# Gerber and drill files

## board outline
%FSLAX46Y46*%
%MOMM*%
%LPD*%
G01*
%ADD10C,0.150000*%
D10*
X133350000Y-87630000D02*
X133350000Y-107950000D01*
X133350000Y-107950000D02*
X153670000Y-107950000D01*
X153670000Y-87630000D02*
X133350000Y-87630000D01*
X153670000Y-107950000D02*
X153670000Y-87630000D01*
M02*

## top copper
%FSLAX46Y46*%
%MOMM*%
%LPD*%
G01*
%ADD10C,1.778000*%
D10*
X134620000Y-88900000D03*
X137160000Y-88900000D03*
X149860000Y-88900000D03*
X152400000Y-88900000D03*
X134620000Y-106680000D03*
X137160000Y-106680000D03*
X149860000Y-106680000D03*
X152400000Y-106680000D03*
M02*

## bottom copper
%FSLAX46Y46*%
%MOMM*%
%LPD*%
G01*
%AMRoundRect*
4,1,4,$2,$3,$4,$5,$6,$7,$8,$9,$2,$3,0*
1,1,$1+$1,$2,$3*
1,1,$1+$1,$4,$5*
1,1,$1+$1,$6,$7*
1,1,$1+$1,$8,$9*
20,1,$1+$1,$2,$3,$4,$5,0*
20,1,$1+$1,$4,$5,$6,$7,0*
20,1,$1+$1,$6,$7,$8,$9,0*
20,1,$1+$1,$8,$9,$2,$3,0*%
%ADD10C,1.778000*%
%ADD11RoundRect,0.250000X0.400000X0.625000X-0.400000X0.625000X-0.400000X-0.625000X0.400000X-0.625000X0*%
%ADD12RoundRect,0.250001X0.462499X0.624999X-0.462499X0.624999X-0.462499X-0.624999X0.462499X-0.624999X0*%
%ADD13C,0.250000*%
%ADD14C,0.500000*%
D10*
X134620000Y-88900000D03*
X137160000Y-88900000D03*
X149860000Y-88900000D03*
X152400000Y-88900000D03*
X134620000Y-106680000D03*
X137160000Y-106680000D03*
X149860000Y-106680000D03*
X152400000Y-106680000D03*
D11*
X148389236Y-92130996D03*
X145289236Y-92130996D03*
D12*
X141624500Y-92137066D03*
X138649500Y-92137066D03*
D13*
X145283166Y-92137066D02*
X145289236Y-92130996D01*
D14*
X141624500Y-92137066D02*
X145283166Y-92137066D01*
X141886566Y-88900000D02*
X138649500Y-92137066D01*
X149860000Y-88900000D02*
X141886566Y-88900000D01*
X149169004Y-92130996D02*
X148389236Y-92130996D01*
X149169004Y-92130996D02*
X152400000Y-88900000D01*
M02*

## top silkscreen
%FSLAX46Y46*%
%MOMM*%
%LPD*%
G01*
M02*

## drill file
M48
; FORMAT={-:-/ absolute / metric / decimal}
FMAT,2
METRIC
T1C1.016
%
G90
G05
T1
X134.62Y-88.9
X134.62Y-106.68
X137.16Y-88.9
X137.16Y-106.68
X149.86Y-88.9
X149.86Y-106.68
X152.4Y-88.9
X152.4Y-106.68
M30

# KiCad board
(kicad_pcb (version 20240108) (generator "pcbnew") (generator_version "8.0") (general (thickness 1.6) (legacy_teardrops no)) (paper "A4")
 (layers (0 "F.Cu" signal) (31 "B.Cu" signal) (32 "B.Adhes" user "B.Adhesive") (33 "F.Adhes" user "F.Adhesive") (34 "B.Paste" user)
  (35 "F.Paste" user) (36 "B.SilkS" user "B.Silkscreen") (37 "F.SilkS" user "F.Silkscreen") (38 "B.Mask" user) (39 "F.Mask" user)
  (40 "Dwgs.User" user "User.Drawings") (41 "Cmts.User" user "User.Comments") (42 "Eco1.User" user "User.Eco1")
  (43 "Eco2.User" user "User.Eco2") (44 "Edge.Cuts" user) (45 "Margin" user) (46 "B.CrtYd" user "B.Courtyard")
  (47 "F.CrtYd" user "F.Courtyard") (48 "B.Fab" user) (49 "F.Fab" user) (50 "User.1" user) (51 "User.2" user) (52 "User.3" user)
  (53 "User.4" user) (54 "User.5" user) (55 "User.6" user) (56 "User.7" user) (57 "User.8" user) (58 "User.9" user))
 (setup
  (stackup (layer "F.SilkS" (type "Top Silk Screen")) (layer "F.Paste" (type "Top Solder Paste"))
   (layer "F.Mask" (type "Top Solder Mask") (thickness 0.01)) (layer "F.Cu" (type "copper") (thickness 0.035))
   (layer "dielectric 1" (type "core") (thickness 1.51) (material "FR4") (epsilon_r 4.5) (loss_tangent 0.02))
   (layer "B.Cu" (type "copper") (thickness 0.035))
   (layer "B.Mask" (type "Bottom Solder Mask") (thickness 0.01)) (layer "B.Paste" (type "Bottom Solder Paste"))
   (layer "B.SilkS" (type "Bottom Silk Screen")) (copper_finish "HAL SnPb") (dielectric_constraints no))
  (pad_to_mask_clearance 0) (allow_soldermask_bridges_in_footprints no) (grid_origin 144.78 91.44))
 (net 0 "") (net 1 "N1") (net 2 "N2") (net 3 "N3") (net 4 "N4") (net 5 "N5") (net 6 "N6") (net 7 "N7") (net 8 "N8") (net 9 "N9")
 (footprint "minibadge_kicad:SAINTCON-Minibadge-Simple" (layer "F.Cu") (at 133.35 87.63)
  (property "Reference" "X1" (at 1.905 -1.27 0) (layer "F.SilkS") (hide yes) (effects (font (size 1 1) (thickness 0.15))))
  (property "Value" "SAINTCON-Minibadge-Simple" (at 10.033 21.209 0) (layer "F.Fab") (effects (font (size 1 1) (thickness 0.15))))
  (fp_line (start 0 0) (end 0 20.32) (stroke (width 0.15) (type solid)) (layer "Edge.Cuts"))
  (fp_line (start 0 20.32) (end 20.32 20.32) (stroke (width 0.15) (type solid)) (layer "Edge.Cuts"))
  (fp_line (start 20.32 0) (end 0 0) (stroke (width 0.15) (type solid)) (layer "Edge.Cuts"))
  (fp_line (start 20.32 20.32) (end 20.32 0) (stroke (width 0.15) (type solid)) (layer "Edge.Cuts"))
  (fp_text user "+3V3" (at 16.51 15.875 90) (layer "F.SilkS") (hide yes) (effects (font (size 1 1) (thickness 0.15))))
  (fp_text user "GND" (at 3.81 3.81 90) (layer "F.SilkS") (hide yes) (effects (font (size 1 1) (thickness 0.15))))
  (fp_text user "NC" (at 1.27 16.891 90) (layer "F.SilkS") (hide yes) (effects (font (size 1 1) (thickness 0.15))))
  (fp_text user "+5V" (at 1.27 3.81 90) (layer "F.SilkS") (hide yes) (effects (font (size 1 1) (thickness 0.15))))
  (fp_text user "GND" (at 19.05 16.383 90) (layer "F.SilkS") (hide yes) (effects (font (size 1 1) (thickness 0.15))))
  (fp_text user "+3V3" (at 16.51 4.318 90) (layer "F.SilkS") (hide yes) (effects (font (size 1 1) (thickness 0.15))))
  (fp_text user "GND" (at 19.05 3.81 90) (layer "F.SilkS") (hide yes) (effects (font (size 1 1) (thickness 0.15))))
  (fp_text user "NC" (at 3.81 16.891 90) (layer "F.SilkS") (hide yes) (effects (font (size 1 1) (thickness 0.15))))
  (pad "1" thru_hole circle (at 1.27 1.27 90) (size 1.778 1.778) (drill 1.016) (layers "*.Cu" "*.Mask") (remove_unused_layers no)
   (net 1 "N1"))
  (pad "2" thru_hole circle (at 3.81 1.27 90) (size 1.778 1.778) (drill 1.016) (layers "*.Cu" "*.Mask") (remove_unused_layers no)
   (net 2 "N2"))
  (pad "7" thru_hole circle (at 16.51 1.27 90) (size 1.778 1.778) (drill 1.016) (layers "*.Cu" "*.Mask") (remove_unused_layers no)
   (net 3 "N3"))
  (pad "8" thru_hole circle (at 19.05 1.27 90) (size 1.778 1.778) (drill 1.016) (layers "*.Cu" "*.Mask") (remove_unused_layers no)
   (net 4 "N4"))
  (pad "9" thru_hole circle (at 1.27 19.05 90) (size 1.778 1.778) (drill 1.016) (layers "*.Cu" "*.Mask") (remove_unused_layers no)
   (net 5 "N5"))
  (pad "10" thru_hole circle (at 3.81 19.05 90) (size 1.778 1.778) (drill 1.016) (layers "*.Cu" "*.Mask") (remove_unused_layers no)
   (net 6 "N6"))
  (pad "15" thru_hole circle (at 16.51 19.05 90) (size 1.778 1.778) (drill 1.016) (layers "*.Cu" "*.Mask") (remove_unused_layers no)
   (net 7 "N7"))
  (pad "16" thru_hole circle (at 19.05 19.05 90) (size 1.778 1.778) (drill 1.016) (layers "*.Cu" "*.Mask") (remove_unused_layers no)
   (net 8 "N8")))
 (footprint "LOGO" (layer "B.Cu") (at 140.131286 90.043)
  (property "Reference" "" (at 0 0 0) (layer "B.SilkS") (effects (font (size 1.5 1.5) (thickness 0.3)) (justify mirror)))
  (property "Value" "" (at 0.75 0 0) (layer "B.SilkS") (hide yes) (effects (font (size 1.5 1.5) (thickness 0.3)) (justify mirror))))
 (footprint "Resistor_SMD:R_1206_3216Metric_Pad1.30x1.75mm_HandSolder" (layer "B.Cu") (at 146.839236 92.130996 180)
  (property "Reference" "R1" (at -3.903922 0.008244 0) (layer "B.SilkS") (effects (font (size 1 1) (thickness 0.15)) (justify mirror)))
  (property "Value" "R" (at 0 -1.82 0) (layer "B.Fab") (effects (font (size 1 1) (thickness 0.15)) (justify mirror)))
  (pad "1" smd roundrect (at -1.55 0 180) (size 1.3 1.75) (layers "B.Cu" "B.Paste" "B.Mask") (roundrect_rratio 0.1923076923) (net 4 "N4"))
  (pad "2" smd roundrect (at 1.55 0 180) (size 1.3 1.75) (layers "B.Cu" "B.Paste" "B.Mask") (roundrect_rratio 0.1923076923) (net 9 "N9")))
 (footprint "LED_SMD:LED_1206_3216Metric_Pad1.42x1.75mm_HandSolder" (layer "B.Cu") (at 140.137 92.137066 180)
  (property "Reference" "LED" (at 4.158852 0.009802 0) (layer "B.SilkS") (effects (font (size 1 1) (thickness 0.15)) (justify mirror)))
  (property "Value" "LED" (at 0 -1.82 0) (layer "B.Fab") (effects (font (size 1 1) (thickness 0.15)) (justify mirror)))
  (pad "1" smd roundrect (at -1.4875 0 180) (size 1.425 1.75) (layers "B.Cu" "B.Paste" "B.Mask") (roundrect_rratio 0.1754392982)
   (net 9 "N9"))
  (pad "2" smd roundrect (at 1.4875 0 180) (size 1.425 1.75) (layers "B.Cu" "B.Paste" "B.Mask") (roundrect_rratio 0.1754392982) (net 3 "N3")))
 (segment (start 145.283166 92.137066) (end 145.289236 92.130996) (width 0.25) (layer "B.Cu") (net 9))
 (segment (start 141.6245 92.137066) (end 145.283166 92.137066) (width 0.5) (layer "B.Cu") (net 9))
 (segment (start 141.886566 88.9) (end 138.6495 92.137066) (width 0.5) (layer "B.Cu") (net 3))
 (segment (start 149.86 88.9) (end 141.886566 88.9) (width 0.5) (layer "B.Cu") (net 3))
 (segment (start 149.169004 92.130996) (end 148.389236 92.130996) (width 0.5) (layer "B.Cu") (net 4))
 (segment (start 149.169004 92.130996) (end 152.4 88.9) (width 0.5) (layer "B.Cu") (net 4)))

